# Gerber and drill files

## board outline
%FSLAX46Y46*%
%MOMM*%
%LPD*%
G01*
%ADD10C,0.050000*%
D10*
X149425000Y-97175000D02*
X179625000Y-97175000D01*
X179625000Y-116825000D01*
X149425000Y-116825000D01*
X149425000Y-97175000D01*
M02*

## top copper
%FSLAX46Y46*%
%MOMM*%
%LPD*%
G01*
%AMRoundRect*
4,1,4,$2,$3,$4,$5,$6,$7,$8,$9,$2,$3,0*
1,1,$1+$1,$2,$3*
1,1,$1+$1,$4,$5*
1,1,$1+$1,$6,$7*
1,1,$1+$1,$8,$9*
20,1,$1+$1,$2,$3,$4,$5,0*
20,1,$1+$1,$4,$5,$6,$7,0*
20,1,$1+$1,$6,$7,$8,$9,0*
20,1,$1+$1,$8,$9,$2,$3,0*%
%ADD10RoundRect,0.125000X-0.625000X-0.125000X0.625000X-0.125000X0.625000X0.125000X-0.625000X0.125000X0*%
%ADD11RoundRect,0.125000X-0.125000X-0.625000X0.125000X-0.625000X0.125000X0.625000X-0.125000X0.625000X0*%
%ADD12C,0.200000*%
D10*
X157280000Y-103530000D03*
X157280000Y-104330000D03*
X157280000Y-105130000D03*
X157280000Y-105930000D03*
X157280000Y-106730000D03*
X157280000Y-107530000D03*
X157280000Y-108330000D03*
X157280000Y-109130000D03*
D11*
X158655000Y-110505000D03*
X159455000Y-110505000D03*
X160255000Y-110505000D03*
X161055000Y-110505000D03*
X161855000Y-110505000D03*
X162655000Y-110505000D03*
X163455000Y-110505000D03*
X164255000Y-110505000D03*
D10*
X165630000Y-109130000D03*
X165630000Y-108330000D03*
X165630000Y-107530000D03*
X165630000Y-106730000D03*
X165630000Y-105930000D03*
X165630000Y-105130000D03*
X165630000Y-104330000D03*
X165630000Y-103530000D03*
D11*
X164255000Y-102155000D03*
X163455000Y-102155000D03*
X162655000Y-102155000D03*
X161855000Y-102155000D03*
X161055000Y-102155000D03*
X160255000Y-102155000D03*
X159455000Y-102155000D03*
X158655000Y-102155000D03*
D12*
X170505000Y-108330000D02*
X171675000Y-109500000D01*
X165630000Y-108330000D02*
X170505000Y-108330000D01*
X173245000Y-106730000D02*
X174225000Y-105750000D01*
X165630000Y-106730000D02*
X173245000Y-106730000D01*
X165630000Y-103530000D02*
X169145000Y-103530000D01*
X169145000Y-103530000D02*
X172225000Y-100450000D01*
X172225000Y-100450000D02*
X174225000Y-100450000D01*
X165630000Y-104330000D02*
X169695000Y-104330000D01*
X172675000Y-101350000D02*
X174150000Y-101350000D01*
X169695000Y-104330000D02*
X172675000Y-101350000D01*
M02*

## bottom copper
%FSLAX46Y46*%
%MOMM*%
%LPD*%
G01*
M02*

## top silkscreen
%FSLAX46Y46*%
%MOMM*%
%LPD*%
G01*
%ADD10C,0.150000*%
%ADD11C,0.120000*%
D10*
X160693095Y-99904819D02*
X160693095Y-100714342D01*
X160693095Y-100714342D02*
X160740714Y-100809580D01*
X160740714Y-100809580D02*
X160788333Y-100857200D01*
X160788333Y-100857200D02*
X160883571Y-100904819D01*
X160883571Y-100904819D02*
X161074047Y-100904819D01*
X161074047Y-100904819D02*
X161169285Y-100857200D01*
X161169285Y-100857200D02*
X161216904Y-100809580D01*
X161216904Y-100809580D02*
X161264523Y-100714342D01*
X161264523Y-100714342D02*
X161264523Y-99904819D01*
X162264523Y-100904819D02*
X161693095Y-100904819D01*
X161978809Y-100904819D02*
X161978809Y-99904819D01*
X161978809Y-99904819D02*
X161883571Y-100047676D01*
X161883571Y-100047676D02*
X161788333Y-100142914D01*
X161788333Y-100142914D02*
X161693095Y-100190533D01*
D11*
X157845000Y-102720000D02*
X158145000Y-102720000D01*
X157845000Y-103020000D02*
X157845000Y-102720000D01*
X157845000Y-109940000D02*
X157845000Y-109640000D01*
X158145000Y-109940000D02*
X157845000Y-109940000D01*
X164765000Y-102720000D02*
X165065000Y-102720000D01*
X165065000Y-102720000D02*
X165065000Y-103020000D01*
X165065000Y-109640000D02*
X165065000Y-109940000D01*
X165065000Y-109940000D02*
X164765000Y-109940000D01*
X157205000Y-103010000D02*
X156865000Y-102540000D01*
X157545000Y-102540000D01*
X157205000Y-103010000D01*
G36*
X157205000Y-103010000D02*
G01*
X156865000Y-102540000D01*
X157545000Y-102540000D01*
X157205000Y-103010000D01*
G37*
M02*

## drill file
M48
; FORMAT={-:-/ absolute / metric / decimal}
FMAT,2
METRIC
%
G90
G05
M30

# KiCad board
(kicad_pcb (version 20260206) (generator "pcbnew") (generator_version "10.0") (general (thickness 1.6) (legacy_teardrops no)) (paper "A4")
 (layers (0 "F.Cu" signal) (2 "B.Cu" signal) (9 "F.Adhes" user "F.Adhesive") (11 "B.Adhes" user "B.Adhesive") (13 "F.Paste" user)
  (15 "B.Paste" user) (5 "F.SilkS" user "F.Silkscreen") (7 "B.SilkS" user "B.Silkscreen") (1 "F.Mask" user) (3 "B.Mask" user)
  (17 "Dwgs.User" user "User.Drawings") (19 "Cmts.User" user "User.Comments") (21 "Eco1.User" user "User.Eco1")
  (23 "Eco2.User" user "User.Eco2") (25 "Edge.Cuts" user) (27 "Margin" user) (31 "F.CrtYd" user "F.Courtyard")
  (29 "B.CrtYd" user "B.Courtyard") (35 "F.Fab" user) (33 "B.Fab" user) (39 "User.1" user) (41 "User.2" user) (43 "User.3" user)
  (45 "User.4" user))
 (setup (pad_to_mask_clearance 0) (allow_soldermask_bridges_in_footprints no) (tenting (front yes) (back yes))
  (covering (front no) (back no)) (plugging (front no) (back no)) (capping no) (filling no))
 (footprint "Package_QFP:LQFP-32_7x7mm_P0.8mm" (layer "F.Cu") (at 161.455 106.33)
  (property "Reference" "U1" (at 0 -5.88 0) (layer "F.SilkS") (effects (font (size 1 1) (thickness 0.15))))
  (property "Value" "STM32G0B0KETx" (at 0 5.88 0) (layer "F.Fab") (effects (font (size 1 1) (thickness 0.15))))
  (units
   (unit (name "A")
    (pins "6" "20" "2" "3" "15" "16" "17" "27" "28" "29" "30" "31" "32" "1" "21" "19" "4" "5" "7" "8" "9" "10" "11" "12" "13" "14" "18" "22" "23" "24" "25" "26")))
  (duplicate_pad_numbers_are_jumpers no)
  (fp_line (start -3.61 -3.61) (end -3.31 -3.61) (stroke (width 0.12) (type solid)) (layer "F.SilkS"))
  (fp_line (start -3.61 -3.31) (end -3.61 -3.61) (stroke (width 0.12) (type solid)) (layer "F.SilkS"))
  (fp_line (start -3.61 3.61) (end -3.61 3.31) (stroke (width 0.12) (type solid)) (layer "F.SilkS"))
  (fp_line (start -3.31 3.61) (end -3.61 3.61) (stroke (width 0.12) (type solid)) (layer "F.SilkS"))
  (fp_line (start 3.31 -3.61) (end 3.61 -3.61) (stroke (width 0.12) (type solid)) (layer "F.SilkS"))
  (fp_line (start 3.61 -3.61) (end 3.61 -3.31) (stroke (width 0.12) (type solid)) (layer "F.SilkS"))
  (fp_line (start 3.61 3.31) (end 3.61 3.61) (stroke (width 0.12) (type solid)) (layer "F.SilkS"))
  (fp_line (start 3.61 3.61) (end 3.31 3.61) (stroke (width 0.12) (type solid)) (layer "F.SilkS"))
  (fp_poly (pts (xy -4.25 -3.32) (xy -4.59 -3.79) (xy -3.91 -3.79)) (stroke (width 0.12) (type solid)) (fill yes) (layer "F.SilkS"))
  (pad "1" smd roundrect (at -4.175 -2.8) (size 1.5 0.5) (layers "F.Cu" "F.Mask" "F.Paste") (roundrect_rratio 0.25)
   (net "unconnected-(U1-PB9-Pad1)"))
  (pad "2" smd roundrect (at -4.175 -2) (size 1.5 0.5) (layers "F.Cu" "F.Mask" "F.Paste") (roundrect_rratio 0.25)
   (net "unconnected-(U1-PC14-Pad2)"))
  (pad "3" smd roundrect (at -4.175 -1.2) (size 1.5 0.5) (layers "F.Cu" "F.Mask" "F.Paste") (roundrect_rratio 0.25)
   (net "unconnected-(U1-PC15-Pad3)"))
  (pad "4" smd roundrect (at -4.175 -0.4) (size 1.5 0.5) (layers "F.Cu" "F.Mask" "F.Paste") (roundrect_rratio 0.25)
   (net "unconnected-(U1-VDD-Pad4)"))
  (pad "5" smd roundrect (at -4.175 0.4) (size 1.5 0.5) (layers "F.Cu" "F.Mask" "F.Paste") (roundrect_rratio 0.25)
   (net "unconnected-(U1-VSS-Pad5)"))
  (pad "6" smd roundrect (at -4.175 1.2) (size 1.5 0.5) (layers "F.Cu" "F.Mask" "F.Paste") (roundrect_rratio 0.25)
   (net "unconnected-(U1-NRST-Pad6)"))
  (pad "7" smd roundrect (at -4.175 2) (size 1.5 0.5) (layers "F.Cu" "F.Mask" "F.Paste") (roundrect_rratio 0.25)
   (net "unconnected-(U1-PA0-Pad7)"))
  (pad "8" smd roundrect (at -4.175 2.8) (size 1.5 0.5) (layers "F.Cu" "F.Mask" "F.Paste") (roundrect_rratio 0.25)
   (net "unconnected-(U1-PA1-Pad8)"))
  (pad "9" smd roundrect (at -2.8 4.175) (size 0.5 1.5) (layers "F.Cu" "F.Mask" "F.Paste") (roundrect_rratio 0.25)
   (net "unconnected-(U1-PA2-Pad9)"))
  (pad "10" smd roundrect (at -2 4.175) (size 0.5 1.5) (layers "F.Cu" "F.Mask" "F.Paste") (roundrect_rratio 0.25)
   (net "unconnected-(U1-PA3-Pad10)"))
  (pad "11" smd roundrect (at -1.2 4.175) (size 0.5 1.5) (layers "F.Cu" "F.Mask" "F.Paste") (roundrect_rratio 0.25)
   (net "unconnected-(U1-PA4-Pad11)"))
  (pad "12" smd roundrect (at -0.4 4.175) (size 0.5 1.5) (layers "F.Cu" "F.Mask" "F.Paste") (roundrect_rratio 0.25)
   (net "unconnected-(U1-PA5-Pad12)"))
  (pad "13" smd roundrect (at 0.4 4.175) (size 0.5 1.5) (layers "F.Cu" "F.Mask" "F.Paste") (roundrect_rratio 0.25)
   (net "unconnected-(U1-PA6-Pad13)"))
  (pad "14" smd roundrect (at 1.2 4.175) (size 0.5 1.5) (layers "F.Cu" "F.Mask" "F.Paste") (roundrect_rratio 0.25)
   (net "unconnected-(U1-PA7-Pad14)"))
  (pad "15" smd roundrect (at 2 4.175) (size 0.5 1.5) (layers "F.Cu" "F.Mask" "F.Paste") (roundrect_rratio 0.25)
   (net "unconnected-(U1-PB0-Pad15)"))
  (pad "16" smd roundrect (at 2.8 4.175) (size 0.5 1.5) (layers "F.Cu" "F.Mask" "F.Paste") (roundrect_rratio 0.25)
   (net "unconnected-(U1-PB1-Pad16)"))
  (pad "17" smd roundrect (at 4.175 2.8) (size 1.5 0.5) (layers "F.Cu" "F.Mask" "F.Paste") (roundrect_rratio 0.25)
   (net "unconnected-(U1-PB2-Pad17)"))
  (pad "18" smd roundrect (at 4.175 2) (size 1.5 0.5) (layers "F.Cu" "F.Mask" "F.Paste") (roundrect_rratio 0.25)
   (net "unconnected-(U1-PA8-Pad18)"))
  (pad "19" smd roundrect (at 4.175 1.2) (size 1.5 0.5) (layers "F.Cu" "F.Mask" "F.Paste") (roundrect_rratio 0.25)
   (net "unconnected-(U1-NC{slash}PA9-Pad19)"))
  (pad "20" smd roundrect (at 4.175 0.4) (size 1.5 0.5) (layers "F.Cu" "F.Mask" "F.Paste") (roundrect_rratio 0.25)
   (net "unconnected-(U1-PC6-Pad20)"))
  (pad "21" smd roundrect (at 4.175 -0.4) (size 1.5 0.5) (layers "F.Cu" "F.Mask" "F.Paste") (roundrect_rratio 0.25)
   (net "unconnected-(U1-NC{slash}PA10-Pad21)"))
  (pad "22" smd roundrect (at 4.175 -1.2) (size 1.5 0.5) (layers "F.Cu" "F.Mask" "F.Paste") (roundrect_rratio 0.25)
   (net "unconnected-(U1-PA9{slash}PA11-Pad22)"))
  (pad "23" smd roundrect (at 4.175 -2) (size 1.5 0.5) (layers "F.Cu" "F.Mask" "F.Paste") (roundrect_rratio 0.25)
   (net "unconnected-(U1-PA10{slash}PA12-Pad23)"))
  (pad "24" smd roundrect (at 4.175 -2.8) (size 1.5 0.5) (layers "F.Cu" "F.Mask" "F.Paste") (roundrect_rratio 0.25)
   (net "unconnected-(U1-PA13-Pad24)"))
  (pad "25" smd roundrect (at 2.8 -4.175) (size 0.5 1.5) (layers "F.Cu" "F.Mask" "F.Paste") (roundrect_rratio 0.25)
   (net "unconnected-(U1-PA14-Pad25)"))
  (pad "26" smd roundrect (at 2 -4.175) (size 0.5 1.5) (layers "F.Cu" "F.Mask" "F.Paste") (roundrect_rratio 0.25)
   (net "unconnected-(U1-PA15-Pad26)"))
  (pad "27" smd roundrect (at 1.2 -4.175) (size 0.5 1.5) (layers "F.Cu" "F.Mask" "F.Paste") (roundrect_rratio 0.25)
   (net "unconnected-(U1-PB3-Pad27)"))
  (pad "28" smd roundrect (at 0.4 -4.175) (size 0.5 1.5) (layers "F.Cu" "F.Mask" "F.Paste") (roundrect_rratio 0.25)
   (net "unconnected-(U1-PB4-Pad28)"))
  (pad "29" smd roundrect (at -0.4 -4.175) (size 0.5 1.5) (layers "F.Cu" "F.Mask" "F.Paste") (roundrect_rratio 0.25)
   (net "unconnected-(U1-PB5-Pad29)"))
  (pad "30" smd roundrect (at -1.2 -4.175) (size 0.5 1.5) (layers "F.Cu" "F.Mask" "F.Paste") (roundrect_rratio 0.25)
   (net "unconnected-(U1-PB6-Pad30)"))
  (pad "31" smd roundrect (at -2 -4.175) (size 0.5 1.5) (layers "F.Cu" "F.Mask" "F.Paste") (roundrect_rratio 0.25)
   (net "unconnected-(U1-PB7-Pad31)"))
  (pad "32" smd roundrect (at -2.8 -4.175) (size 0.5 1.5) (layers "F.Cu" "F.Mask" "F.Paste") (roundrect_rratio 0.25)
   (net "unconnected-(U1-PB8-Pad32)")))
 (gr_rect (start 149.425 97.175) (end 179.625 116.825) (stroke (width 0.05) (type default)) (fill no) (layer "Edge.Cuts"))
 (segment (start 170.505 108.33) (end 171.675 109.5) (width 0.2) (layer "F.Cu") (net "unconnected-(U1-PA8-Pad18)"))
 (segment (start 165.63 108.33) (end 170.505 108.33) (width 0.2) (layer "F.Cu") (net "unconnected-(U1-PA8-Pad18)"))
 (segment (start 173.245 106.73) (end 174.225 105.75) (width 0.2) (layer "F.Cu") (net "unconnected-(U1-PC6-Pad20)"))
 (segment (start 165.63 106.73) (end 173.245 106.73) (width 0.2) (layer "F.Cu") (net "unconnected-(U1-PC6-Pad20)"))
 (segment (start 165.63 103.53) (end 169.145 103.53) (width 0.2) (layer "F.Cu") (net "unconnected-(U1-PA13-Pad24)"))
 (segment (start 169.145 103.53) (end 172.225 100.45) (width 0.2) (layer "F.Cu") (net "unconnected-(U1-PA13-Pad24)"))
 (segment (start 172.225 100.45) (end 174.225 100.45) (width 0.2) (layer "F.Cu") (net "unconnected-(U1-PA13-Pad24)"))
 (segment (start 165.63 104.33) (end 169.695 104.33) (width 0.2) (layer "F.Cu") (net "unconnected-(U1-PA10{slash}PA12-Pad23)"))
 (segment (start 172.675 101.35) (end 174.15 101.35) (width 0.2) (layer "F.Cu") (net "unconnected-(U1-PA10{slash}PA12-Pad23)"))
 (segment (start 169.695 104.33) (end 172.675 101.35) (width 0.2) (layer "F.Cu") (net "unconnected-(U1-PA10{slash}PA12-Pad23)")))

